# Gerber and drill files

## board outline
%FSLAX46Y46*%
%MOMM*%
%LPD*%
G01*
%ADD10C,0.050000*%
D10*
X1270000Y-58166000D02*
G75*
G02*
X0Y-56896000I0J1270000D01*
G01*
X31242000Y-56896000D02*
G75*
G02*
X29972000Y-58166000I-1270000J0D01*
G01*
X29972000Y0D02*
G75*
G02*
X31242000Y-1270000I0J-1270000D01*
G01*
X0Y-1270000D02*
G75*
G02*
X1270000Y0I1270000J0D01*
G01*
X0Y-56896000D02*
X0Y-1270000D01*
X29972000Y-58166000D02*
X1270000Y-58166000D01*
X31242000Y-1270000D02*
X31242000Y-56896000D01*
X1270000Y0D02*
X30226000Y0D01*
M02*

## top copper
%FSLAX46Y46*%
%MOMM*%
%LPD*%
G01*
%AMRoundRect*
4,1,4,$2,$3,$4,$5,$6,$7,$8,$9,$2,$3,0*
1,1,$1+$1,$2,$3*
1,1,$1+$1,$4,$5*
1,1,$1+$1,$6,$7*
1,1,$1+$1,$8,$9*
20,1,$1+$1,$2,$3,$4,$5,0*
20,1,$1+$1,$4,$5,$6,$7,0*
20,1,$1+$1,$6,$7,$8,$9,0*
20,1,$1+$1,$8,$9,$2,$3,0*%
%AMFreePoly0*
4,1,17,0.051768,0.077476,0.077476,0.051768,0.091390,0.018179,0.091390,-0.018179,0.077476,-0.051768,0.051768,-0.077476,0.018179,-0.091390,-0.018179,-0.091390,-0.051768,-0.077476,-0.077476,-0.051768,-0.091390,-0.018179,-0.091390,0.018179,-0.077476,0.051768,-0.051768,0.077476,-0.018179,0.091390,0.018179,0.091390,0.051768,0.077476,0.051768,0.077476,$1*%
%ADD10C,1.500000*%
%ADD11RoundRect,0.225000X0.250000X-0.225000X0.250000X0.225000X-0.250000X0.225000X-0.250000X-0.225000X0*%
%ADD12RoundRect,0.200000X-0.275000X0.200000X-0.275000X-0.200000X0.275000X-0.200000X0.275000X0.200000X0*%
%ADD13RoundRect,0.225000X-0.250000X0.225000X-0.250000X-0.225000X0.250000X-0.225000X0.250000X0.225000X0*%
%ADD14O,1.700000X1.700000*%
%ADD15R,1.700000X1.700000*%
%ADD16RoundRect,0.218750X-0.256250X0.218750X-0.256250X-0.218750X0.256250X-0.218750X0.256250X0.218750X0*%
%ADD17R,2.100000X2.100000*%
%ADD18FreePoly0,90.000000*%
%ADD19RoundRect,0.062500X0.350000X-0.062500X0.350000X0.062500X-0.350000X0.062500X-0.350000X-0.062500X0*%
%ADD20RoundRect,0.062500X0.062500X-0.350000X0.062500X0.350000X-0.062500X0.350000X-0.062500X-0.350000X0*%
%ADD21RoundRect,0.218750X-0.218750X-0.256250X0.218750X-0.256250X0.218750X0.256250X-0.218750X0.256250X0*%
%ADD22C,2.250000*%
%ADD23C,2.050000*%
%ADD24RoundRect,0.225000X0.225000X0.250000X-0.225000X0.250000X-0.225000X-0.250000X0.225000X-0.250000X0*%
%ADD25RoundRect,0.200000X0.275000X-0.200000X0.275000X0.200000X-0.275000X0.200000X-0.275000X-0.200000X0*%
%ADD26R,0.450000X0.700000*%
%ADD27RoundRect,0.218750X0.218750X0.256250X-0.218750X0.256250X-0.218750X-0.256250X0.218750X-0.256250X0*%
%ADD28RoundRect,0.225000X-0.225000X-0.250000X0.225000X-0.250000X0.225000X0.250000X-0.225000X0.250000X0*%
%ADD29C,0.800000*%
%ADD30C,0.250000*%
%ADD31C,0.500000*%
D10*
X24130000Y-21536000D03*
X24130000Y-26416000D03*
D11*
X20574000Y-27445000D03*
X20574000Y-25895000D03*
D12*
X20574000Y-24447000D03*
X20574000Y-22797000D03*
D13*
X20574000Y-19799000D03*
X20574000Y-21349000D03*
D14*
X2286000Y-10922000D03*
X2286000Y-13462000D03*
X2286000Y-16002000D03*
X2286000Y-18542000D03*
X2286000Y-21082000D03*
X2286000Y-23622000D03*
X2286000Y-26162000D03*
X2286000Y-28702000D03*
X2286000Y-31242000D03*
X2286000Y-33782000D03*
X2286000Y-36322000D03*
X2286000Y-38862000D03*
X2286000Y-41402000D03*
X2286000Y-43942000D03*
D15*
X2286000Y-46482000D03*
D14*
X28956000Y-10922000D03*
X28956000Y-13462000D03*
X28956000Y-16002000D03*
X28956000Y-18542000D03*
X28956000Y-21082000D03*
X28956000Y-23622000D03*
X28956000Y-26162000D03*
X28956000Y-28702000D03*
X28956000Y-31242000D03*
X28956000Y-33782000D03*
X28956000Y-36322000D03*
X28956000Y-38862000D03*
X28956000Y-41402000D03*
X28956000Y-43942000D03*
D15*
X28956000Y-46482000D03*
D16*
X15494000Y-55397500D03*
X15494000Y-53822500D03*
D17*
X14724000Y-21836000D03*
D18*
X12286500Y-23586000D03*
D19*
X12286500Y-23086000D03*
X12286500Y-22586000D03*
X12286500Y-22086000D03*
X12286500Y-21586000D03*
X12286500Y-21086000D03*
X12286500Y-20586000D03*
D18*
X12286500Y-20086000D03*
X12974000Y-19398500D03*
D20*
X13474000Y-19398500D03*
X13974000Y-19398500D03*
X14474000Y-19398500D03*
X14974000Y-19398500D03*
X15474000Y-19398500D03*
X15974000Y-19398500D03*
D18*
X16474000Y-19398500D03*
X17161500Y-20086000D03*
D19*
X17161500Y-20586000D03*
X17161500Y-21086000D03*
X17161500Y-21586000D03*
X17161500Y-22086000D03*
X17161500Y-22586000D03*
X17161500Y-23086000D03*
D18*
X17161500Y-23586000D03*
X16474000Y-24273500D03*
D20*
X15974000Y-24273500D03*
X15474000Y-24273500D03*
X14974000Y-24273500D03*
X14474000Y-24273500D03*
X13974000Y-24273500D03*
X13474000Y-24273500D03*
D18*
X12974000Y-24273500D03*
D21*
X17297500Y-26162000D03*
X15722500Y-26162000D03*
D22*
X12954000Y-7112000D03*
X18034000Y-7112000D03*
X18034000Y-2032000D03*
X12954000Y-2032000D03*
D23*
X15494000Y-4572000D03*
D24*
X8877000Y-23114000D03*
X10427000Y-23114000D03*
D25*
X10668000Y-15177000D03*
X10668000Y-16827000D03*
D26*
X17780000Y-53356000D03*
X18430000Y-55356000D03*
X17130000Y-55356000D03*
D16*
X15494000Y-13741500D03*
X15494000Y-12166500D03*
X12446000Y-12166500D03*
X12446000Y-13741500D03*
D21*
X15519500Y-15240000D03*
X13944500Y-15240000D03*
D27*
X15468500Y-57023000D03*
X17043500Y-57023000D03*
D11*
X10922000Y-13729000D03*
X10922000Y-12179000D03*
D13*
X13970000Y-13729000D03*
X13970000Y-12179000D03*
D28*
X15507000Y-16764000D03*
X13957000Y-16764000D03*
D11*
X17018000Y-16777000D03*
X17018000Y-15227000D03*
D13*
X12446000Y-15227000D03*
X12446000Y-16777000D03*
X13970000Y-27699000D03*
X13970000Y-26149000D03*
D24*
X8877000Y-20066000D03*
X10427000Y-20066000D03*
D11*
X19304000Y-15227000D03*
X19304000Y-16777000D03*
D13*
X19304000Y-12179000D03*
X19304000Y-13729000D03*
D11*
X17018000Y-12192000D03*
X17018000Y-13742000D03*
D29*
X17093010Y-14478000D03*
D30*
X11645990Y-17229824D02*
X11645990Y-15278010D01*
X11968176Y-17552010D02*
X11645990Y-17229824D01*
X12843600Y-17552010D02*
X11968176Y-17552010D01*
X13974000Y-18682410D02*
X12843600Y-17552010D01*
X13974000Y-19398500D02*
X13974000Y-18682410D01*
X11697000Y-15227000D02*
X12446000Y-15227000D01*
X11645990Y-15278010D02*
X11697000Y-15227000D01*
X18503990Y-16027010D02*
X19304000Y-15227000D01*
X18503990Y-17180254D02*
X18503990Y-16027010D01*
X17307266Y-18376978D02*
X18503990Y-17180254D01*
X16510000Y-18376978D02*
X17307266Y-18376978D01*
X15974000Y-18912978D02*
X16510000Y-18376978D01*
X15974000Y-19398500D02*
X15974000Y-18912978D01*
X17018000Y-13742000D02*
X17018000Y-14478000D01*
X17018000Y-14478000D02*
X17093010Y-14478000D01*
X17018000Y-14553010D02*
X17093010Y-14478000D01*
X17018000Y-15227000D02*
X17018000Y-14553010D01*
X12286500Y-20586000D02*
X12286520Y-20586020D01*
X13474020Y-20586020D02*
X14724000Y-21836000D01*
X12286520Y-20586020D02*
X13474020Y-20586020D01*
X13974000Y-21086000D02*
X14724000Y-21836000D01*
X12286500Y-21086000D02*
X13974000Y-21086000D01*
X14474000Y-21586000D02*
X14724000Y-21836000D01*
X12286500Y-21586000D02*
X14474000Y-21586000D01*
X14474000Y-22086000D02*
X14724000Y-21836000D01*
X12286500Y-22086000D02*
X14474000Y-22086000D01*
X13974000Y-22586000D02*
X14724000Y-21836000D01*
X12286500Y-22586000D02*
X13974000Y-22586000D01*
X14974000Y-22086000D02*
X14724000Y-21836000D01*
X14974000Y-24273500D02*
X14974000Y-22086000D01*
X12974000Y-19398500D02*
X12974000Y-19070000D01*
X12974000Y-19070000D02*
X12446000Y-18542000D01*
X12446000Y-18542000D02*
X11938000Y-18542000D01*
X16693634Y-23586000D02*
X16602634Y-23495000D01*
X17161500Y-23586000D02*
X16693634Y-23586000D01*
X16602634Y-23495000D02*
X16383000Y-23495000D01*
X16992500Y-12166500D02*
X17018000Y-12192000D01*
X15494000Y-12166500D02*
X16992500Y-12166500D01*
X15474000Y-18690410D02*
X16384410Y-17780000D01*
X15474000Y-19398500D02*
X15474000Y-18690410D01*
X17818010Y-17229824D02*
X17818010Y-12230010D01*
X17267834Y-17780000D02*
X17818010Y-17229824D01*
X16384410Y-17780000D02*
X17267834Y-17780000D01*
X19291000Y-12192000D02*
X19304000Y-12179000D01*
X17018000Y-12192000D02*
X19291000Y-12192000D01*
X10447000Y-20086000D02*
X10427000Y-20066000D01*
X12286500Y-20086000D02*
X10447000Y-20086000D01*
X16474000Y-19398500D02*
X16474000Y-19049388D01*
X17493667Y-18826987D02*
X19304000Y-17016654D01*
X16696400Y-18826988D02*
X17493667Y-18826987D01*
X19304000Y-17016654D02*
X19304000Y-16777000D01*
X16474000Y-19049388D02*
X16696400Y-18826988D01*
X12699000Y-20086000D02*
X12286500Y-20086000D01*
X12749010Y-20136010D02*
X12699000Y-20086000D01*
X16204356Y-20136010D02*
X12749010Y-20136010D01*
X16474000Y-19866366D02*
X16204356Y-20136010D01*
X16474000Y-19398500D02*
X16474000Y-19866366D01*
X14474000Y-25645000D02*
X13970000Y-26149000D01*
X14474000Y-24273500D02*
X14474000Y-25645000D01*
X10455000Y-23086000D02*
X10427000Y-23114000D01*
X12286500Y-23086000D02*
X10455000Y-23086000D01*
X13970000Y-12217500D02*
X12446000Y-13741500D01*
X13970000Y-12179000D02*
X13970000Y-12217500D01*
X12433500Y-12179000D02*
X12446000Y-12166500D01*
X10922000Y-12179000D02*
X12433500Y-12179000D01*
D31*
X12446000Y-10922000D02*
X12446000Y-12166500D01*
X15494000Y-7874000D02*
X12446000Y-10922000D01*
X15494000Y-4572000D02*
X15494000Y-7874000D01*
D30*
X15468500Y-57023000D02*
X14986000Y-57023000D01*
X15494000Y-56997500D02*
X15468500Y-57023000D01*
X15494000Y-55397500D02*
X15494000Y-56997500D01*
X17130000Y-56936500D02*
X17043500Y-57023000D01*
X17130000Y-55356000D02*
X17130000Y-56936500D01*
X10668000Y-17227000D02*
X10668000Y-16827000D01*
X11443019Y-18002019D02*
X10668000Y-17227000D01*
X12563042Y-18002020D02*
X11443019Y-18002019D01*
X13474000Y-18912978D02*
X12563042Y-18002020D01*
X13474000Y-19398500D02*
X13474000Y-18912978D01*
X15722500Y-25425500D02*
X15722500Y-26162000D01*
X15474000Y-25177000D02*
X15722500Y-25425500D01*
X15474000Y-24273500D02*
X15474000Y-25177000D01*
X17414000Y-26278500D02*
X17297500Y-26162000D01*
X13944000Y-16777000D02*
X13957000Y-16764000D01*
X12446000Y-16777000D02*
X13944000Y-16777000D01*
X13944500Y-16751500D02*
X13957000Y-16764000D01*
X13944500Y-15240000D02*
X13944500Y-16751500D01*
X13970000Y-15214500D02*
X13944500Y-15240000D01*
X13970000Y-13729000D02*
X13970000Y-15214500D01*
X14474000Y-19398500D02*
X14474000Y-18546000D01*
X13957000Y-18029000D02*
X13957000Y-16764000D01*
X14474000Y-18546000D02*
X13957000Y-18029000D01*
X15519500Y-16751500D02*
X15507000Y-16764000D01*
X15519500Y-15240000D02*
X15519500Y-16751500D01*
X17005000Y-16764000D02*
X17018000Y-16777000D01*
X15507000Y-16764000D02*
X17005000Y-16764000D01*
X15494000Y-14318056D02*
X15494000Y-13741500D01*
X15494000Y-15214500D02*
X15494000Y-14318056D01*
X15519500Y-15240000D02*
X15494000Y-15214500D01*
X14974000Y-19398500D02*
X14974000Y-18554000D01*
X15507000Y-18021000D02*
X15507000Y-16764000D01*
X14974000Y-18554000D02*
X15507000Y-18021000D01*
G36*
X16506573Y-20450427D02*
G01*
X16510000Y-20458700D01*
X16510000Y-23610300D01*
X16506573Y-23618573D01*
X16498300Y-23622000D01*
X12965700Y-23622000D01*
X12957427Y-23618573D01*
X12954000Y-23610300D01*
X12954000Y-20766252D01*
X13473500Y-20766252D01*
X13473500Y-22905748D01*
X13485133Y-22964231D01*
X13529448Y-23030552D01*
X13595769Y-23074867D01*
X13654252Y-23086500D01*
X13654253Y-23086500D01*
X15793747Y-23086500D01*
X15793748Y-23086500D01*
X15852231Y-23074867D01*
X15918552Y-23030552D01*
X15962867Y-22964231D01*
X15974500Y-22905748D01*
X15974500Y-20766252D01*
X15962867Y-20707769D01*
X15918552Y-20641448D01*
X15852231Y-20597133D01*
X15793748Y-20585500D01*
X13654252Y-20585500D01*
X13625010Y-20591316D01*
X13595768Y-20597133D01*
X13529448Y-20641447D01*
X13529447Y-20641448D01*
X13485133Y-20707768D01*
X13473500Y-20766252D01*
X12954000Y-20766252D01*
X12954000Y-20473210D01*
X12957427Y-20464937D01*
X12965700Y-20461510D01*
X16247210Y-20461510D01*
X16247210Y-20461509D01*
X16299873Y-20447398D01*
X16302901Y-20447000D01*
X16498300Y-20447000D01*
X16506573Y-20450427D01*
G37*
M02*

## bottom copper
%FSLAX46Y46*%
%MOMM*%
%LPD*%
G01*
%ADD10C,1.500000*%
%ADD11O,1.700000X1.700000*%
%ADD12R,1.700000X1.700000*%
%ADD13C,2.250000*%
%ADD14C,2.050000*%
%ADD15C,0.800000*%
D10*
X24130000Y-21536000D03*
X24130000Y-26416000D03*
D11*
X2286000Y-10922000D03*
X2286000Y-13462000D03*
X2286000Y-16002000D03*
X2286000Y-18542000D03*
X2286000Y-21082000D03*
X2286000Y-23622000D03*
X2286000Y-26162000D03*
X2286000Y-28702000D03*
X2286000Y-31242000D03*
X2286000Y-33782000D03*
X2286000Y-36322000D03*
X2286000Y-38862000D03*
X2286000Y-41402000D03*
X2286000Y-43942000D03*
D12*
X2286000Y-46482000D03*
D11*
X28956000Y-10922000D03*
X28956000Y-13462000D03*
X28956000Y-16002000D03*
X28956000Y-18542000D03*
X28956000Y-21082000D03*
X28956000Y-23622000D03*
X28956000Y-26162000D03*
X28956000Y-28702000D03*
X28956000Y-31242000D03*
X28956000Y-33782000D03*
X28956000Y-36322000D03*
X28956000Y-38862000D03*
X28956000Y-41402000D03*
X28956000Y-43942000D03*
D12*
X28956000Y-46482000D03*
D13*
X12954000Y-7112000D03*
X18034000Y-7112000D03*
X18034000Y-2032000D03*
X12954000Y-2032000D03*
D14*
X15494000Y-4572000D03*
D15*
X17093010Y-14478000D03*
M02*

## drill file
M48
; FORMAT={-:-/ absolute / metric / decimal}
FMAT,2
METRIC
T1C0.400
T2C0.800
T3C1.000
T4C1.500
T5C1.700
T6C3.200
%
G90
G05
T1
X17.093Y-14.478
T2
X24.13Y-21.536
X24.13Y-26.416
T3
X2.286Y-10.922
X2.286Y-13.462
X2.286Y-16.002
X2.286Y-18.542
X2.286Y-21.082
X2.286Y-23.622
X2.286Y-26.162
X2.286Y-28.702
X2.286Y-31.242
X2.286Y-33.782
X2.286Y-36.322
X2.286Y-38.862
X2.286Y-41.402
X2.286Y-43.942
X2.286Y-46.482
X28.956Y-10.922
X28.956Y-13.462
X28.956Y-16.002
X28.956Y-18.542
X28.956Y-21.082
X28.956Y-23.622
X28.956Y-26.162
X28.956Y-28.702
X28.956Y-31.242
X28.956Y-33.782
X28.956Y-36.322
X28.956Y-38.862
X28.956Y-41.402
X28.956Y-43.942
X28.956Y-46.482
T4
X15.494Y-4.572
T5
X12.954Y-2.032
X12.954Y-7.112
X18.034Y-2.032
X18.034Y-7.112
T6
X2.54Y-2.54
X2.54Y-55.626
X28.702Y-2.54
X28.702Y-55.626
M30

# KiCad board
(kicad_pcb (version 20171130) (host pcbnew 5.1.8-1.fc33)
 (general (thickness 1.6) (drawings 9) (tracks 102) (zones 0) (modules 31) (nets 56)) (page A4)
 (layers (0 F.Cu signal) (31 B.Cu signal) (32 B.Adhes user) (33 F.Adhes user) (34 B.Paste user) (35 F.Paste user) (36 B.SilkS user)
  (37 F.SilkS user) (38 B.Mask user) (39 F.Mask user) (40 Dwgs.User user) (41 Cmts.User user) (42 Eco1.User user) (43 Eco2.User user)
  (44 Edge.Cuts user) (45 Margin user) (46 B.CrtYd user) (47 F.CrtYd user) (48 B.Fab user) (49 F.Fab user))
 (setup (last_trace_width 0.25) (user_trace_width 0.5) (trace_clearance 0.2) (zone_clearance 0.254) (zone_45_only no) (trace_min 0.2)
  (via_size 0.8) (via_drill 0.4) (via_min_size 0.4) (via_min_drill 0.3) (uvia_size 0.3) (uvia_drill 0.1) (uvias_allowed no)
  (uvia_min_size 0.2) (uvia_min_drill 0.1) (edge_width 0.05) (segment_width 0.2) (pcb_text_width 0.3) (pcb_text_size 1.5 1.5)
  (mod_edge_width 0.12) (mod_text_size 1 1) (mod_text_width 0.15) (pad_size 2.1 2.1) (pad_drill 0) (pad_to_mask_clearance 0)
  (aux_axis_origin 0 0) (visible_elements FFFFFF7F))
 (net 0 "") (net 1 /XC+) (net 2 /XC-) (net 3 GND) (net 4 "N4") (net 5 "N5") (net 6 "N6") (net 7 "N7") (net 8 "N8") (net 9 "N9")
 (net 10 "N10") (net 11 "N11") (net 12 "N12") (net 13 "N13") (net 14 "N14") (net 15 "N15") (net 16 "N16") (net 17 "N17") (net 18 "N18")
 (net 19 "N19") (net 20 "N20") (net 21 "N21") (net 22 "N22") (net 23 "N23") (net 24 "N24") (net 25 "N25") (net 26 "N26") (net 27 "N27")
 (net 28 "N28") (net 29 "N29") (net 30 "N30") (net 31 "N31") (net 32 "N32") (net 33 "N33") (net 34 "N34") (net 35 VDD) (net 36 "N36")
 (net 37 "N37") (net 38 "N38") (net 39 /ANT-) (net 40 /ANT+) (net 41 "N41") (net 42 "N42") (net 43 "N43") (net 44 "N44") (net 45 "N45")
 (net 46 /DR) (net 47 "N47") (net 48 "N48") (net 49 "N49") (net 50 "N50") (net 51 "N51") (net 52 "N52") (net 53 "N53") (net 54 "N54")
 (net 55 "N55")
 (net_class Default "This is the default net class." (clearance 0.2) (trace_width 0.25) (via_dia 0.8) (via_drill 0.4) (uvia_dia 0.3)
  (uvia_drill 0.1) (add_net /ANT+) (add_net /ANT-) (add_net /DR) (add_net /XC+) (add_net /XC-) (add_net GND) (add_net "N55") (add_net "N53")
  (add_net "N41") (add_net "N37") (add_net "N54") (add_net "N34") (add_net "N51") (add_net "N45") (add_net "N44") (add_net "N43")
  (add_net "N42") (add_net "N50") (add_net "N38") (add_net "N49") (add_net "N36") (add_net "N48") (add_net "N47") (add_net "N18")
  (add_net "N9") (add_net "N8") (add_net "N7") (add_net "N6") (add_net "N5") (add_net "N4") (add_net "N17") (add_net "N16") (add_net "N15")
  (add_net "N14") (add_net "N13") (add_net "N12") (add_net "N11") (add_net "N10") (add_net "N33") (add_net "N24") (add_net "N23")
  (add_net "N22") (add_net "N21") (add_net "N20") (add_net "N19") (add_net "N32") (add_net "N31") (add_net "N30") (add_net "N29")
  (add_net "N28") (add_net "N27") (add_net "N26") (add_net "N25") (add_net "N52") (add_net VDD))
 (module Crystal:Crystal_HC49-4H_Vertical (layer F.Cu) (at 24.13 26.416 90)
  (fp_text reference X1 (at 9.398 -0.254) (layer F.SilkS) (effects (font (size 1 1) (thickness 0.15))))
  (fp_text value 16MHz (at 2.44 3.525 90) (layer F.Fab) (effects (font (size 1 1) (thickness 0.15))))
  (pad 2 thru_hole circle (at 4.88 0 90) (size 1.5 1.5) (drill 0.8) (layers *.Cu *.Mask) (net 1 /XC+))
  (pad 1 thru_hole circle (at 0 0 90) (size 1.5 1.5) (drill 0.8) (layers *.Cu *.Mask) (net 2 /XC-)))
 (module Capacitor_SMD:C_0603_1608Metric (layer F.Cu) (at 20.574 26.67 90)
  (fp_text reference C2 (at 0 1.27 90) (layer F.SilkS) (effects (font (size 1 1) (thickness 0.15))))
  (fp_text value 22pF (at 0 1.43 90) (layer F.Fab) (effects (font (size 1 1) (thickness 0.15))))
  (pad 1 smd roundrect (at -0.775 0 90) (size 0.9 0.95) (layers F.Cu F.Paste F.Mask) (roundrect_rratio 0.25) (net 1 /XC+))
  (pad 2 smd roundrect (at 0.775 0 90) (size 0.9 0.95) (layers F.Cu F.Paste F.Mask) (roundrect_rratio 0.25) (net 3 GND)))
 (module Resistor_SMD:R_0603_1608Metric (layer F.Cu) (at 20.574 23.622 270)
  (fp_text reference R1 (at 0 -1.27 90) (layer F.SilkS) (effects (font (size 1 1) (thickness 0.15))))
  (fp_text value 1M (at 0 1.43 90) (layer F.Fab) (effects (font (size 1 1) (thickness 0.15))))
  (pad 2 smd roundrect (at 0.825 0 270) (size 0.8 0.95) (layers F.Cu F.Paste F.Mask) (roundrect_rratio 0.25) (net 2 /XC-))
  (pad 1 smd roundrect (at -0.825 0 270) (size 0.8 0.95) (layers F.Cu F.Paste F.Mask) (roundrect_rratio 0.25) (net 1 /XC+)))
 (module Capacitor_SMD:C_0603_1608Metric (layer F.Cu) (at 20.574 20.574 270)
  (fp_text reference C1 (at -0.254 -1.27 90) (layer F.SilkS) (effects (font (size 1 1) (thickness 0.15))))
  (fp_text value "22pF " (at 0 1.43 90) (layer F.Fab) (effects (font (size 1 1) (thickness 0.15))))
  (pad 1 smd roundrect (at -0.775 0 270) (size 0.9 0.95) (layers F.Cu F.Paste F.Mask) (roundrect_rratio 0.25) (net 2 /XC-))
  (pad 2 smd roundrect (at 0.775 0 270) (size 0.9 0.95) (layers F.Cu F.Paste F.Mask) (roundrect_rratio 0.25) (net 3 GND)))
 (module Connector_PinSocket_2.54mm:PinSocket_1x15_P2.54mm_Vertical (layer F.Cu) (at 2.286 46.482 180)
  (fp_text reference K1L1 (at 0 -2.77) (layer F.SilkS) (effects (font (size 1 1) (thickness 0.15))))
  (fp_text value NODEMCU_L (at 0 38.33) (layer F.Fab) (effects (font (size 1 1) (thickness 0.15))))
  (pad 15 thru_hole oval (at 0 35.56 180) (size 1.7 1.7) (drill 1) (layers *.Cu *.Mask) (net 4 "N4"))
  (pad 14 thru_hole oval (at 0 33.02 180) (size 1.7 1.7) (drill 1) (layers *.Cu *.Mask) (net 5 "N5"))
  (pad 13 thru_hole oval (at 0 30.48 180) (size 1.7 1.7) (drill 1) (layers *.Cu *.Mask) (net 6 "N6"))
  (pad 12 thru_hole oval (at 0 27.94 180) (size 1.7 1.7) (drill 1) (layers *.Cu *.Mask) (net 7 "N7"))
  (pad 11 thru_hole oval (at 0 25.4 180) (size 1.7 1.7) (drill 1) (layers *.Cu *.Mask) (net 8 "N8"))
  (pad 10 thru_hole oval (at 0 22.86 180) (size 1.7 1.7) (drill 1) (layers *.Cu *.Mask) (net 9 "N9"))
  (pad 9 thru_hole oval (at 0 20.32 180) (size 1.7 1.7) (drill 1) (layers *.Cu *.Mask) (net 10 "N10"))
  (pad 8 thru_hole oval (at 0 17.78 180) (size 1.7 1.7) (drill 1) (layers *.Cu *.Mask) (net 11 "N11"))
  (pad 7 thru_hole oval (at 0 15.24 180) (size 1.7 1.7) (drill 1) (layers *.Cu *.Mask) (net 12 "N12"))
  (pad 6 thru_hole oval (at 0 12.7 180) (size 1.7 1.7) (drill 1) (layers *.Cu *.Mask) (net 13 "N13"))
  (pad 5 thru_hole oval (at 0 10.16 180) (size 1.7 1.7) (drill 1) (layers *.Cu *.Mask) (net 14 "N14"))
  (pad 4 thru_hole oval (at 0 7.62 180) (size 1.7 1.7) (drill 1) (layers *.Cu *.Mask) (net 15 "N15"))
  (pad 3 thru_hole oval (at 0 5.08 180) (size 1.7 1.7) (drill 1) (layers *.Cu *.Mask) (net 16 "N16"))
  (pad 2 thru_hole oval (at 0 2.54 180) (size 1.7 1.7) (drill 1) (layers *.Cu *.Mask) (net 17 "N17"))
  (pad 1 thru_hole rect (at 0 0 180) (size 1.7 1.7) (drill 1) (layers *.Cu *.Mask) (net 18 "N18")))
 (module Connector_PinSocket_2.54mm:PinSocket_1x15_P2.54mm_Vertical (layer F.Cu) (at 28.956 46.482 180)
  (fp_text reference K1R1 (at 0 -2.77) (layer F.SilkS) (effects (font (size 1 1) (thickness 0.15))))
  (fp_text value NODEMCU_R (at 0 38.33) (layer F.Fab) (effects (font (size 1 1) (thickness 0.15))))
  (pad 15 thru_hole oval (at 0 35.56 180) (size 1.7 1.7) (drill 1) (layers *.Cu *.Mask) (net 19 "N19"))
  (pad 14 thru_hole oval (at 0 33.02 180) (size 1.7 1.7) (drill 1) (layers *.Cu *.Mask) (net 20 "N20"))
  (pad 13 thru_hole oval (at 0 30.48 180) (size 1.7 1.7) (drill 1) (layers *.Cu *.Mask) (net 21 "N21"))
  (pad 12 thru_hole oval (at 0 27.94 180) (size 1.7 1.7) (drill 1) (layers *.Cu *.Mask) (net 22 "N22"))
  (pad 11 thru_hole oval (at 0 25.4 180) (size 1.7 1.7) (drill 1) (layers *.Cu *.Mask) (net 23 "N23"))
  (pad 10 thru_hole oval (at 0 22.86 180) (size 1.7 1.7) (drill 1) (layers *.Cu *.Mask) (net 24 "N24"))
  (pad 9 thru_hole oval (at 0 20.32 180) (size 1.7 1.7) (drill 1) (layers *.Cu *.Mask) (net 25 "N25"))
  (pad 8 thru_hole oval (at 0 17.78 180) (size 1.7 1.7) (drill 1) (layers *.Cu *.Mask) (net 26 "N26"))
  (pad 7 thru_hole oval (at 0 15.24 180) (size 1.7 1.7) (drill 1) (layers *.Cu *.Mask) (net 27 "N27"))
  (pad 6 thru_hole oval (at 0 12.7 180) (size 1.7 1.7) (drill 1) (layers *.Cu *.Mask) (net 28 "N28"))
  (pad 5 thru_hole oval (at 0 10.16 180) (size 1.7 1.7) (drill 1) (layers *.Cu *.Mask) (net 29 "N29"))
  (pad 4 thru_hole oval (at 0 7.62 180) (size 1.7 1.7) (drill 1) (layers *.Cu *.Mask) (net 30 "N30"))
  (pad 3 thru_hole oval (at 0 5.08 180) (size 1.7 1.7) (drill 1) (layers *.Cu *.Mask) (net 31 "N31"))
  (pad 2 thru_hole oval (at 0 2.54 180) (size 1.7 1.7) (drill 1) (layers *.Cu *.Mask) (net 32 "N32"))
  (pad 1 thru_hole rect (at 0 0 180) (size 1.7 1.7) (drill 1) (layers *.Cu *.Mask) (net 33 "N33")))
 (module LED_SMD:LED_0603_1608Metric (layer F.Cu) (at 15.494 54.61 270)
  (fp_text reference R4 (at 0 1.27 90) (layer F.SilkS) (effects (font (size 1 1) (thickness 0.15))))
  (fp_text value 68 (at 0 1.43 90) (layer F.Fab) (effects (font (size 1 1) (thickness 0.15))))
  (pad 2 smd roundrect (at 0.7875 0 270) (size 0.875 0.95) (layers F.Cu F.Paste F.Mask) (roundrect_rratio 0.25) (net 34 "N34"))
  (pad 1 smd roundrect (at -0.7875 0 270) (size 0.875 0.95) (layers F.Cu F.Paste F.Mask) (roundrect_rratio 0.25) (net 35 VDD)))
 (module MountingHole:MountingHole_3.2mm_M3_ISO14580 (layer F.Cu) (at 2.54 55.626)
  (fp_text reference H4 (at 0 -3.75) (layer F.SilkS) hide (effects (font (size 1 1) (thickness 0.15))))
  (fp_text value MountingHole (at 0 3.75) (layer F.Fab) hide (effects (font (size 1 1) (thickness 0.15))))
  (pad 1 np_thru_hole circle (at 0 0) (size 3.2 3.2) (drill 3.2) (layers *.Cu *.Mask)))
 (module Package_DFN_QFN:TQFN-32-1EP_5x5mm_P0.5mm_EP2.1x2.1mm (layer F.Cu) (at 14.724 21.836 90)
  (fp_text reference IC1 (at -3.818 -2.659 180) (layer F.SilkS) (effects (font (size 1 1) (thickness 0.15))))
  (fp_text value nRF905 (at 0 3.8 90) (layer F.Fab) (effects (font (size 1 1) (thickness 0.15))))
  (pad "" smd roundrect (at 0.525 0.525 90) (size 0.85 0.85) (layers F.Paste) (roundrect_rratio 0.25))
  (pad "" smd roundrect (at 0.525 -0.525 90) (size 0.85 0.85) (layers F.Paste) (roundrect_rratio 0.25))
  (pad "" smd roundrect (at -0.525 0.525 90) (size 0.85 0.85) (layers F.Paste) (roundrect_rratio 0.25))
  (pad "" smd roundrect (at -0.525 -0.525 90) (size 0.85 0.85) (layers F.Paste) (roundrect_rratio 0.25))
  (pad 33 smd rect (at 0 0 90) (size 2.1 2.1) (layers F.Cu F.Mask))
  (pad 32 smd custom (at -1.75 -2.4375 90) (size 0.18636 0.18636) (layers F.Cu F.Paste F.Mask) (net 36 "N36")
   (options (clearance outline) (anchor circle)) (primitives))
  (pad 31 smd roundrect (at -1.25 -2.4375 90) (size 0.25 0.825) (layers F.Cu F.Paste F.Mask) (roundrect_rratio 0.25) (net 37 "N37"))
  (pad 30 smd roundrect (at -0.75 -2.4375 90) (size 0.25 0.825) (layers F.Cu F.Paste F.Mask) (roundrect_rratio 0.25) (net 3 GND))
  (pad 29 smd roundrect (at -0.25 -2.4375 90) (size 0.25 0.825) (layers F.Cu F.Paste F.Mask) (roundrect_rratio 0.25) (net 3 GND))
  (pad 28 smd roundrect (at 0.25 -2.4375 90) (size 0.25 0.825) (layers F.Cu F.Paste F.Mask) (roundrect_rratio 0.25) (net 3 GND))
  (pad 27 smd roundrect (at 0.75 -2.4375 90) (size 0.25 0.825) (layers F.Cu F.Paste F.Mask) (roundrect_rratio 0.25) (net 3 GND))
  (pad 26 smd roundrect (at 1.25 -2.4375 90) (size 0.25 0.825) (layers F.Cu F.Paste F.Mask) (roundrect_rratio 0.25) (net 3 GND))
  (pad 25 smd custom (at 1.75 -2.4375 90) (size 0.18636 0.18636) (layers F.Cu F.Paste F.Mask) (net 35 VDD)
   (options (clearance outline) (anchor circle)) (primitives))
  (pad 24 smd custom (at 2.4375 -1.75 90) (size 0.18636 0.18636) (layers F.Cu F.Paste F.Mask) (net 3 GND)
   (options (clearance outline) (anchor circle)) (primitives))
  (pad 23 smd roundrect (at 2.4375 -1.25 90) (size 0.825 0.25) (layers F.Cu F.Paste F.Mask) (roundrect_rratio 0.25) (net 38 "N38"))
  (pad 22 smd roundrect (at 2.4375 -0.75 90) (size 0.825 0.25) (layers F.Cu F.Paste F.Mask) (roundrect_rratio 0.25) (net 3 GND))
  (pad 21 smd roundrect (at 2.4375 -0.25 90) (size 0.825 0.25) (layers F.Cu F.Paste F.Mask) (roundrect_rratio 0.25) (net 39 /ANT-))
  (pad 20 smd roundrect (at 2.4375 0.25 90) (size 0.825 0.25) (layers F.Cu F.Paste F.Mask) (roundrect_rratio 0.25) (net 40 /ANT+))
  (pad 19 smd roundrect (at 2.4375 0.75 90) (size 0.825 0.25) (layers F.Cu F.Paste F.Mask) (roundrect_rratio 0.25) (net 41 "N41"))
  (pad 18 smd roundrect (at 2.4375 1.25 90) (size 0.825 0.25) (layers F.Cu F.Paste F.Mask) (roundrect_rratio 0.25) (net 3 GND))
  (pad 17 smd custom (at 2.4375 1.75 90) (size 0.18636 0.18636) (layers F.Cu F.Paste F.Mask) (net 35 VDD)
   (options (clearance outline) (anchor circle)) (primitives))
  (pad 16 smd custom (at 1.75 2.4375 90) (size 0.18636 0.18636) (layers F.Cu F.Paste F.Mask) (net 3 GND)
   (options (clearance outline) (anchor circle)) (primitives))
  (pad 15 smd roundrect (at 1.25 2.4375 90) (size 0.25 0.825) (layers F.Cu F.Paste F.Mask) (roundrect_rratio 0.25) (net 2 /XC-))
  (pad 14 smd roundrect (at 0.75 2.4375 90) (size 0.25 0.825) (layers F.Cu F.Paste F.Mask) (roundrect_rratio 0.25) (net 1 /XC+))
  (pad 13 smd roundrect (at 0.25 2.4375 90) (size 0.25 0.825) (layers F.Cu F.Paste F.Mask) (roundrect_rratio 0.25) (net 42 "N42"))
  (pad 12 smd roundrect (at -0.25 2.4375 90) (size 0.25 0.825) (layers F.Cu F.Paste F.Mask) (roundrect_rratio 0.25) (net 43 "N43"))
  (pad 11 smd roundrect (at -0.75 2.4375 90) (size 0.25 0.825) (layers F.Cu F.Paste F.Mask) (roundrect_rratio 0.25) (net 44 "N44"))
  (pad 10 smd roundrect (at -1.25 2.4375 90) (size 0.25 0.825) (layers F.Cu F.Paste F.Mask) (roundrect_rratio 0.25) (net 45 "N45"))
  (pad 9 smd custom (at -1.75 2.4375 90) (size 0.18636 0.18636) (layers F.Cu F.Paste F.Mask) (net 3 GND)
   (options (clearance outline) (anchor circle)) (primitives))
  (pad 8 smd custom (at -2.4375 1.75 90) (size 0.18636 0.18636) (layers F.Cu F.Paste F.Mask) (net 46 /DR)
   (options (clearance outline) (anchor circle)) (primitives))
  (pad 7 smd roundrect (at -2.4375 1.25 90) (size 0.825 0.25) (layers F.Cu F.Paste F.Mask) (roundrect_rratio 0.25) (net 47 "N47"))
  (pad 6 smd roundrect (at -2.4375 0.75 90) (size 0.825 0.25) (layers F.Cu F.Paste F.Mask) (roundrect_rratio 0.25) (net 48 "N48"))
  (pad 5 smd roundrect (at -2.4375 0.25 90) (size 0.825 0.25) (layers F.Cu F.Paste F.Mask) (roundrect_rratio 0.25) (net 3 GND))
  (pad 4 smd roundrect (at -2.4375 -0.25 90) (size 0.825 0.25) (layers F.Cu F.Paste F.Mask) (roundrect_rratio 0.25) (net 35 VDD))
  (pad 3 smd roundrect (at -2.4375 -0.75 90) (size 0.825 0.25) (layers F.Cu F.Paste F.Mask) (roundrect_rratio 0.25) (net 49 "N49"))
  (pad 2 smd roundrect (at -2.4375 -1.25 90) (size 0.825 0.25) (layers F.Cu F.Paste F.Mask) (roundrect_rratio 0.25) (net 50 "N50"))
  (pad 1 smd custom (at -2.4375 -1.75 90) (size 0.18636 0.18636) (layers F.Cu F.Paste F.Mask) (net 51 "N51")
   (options (clearance outline) (anchor circle)) (primitives)))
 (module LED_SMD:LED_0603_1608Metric (layer F.Cu) (at 16.51 26.162)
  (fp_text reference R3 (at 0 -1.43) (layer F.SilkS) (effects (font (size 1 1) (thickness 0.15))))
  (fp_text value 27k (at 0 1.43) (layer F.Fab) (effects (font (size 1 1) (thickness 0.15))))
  (pad 2 smd roundrect (at 0.7875 0) (size 0.875 0.95) (layers F.Cu F.Paste F.Mask) (roundrect_rratio 0.25) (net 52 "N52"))
  (pad 1 smd roundrect (at -0.7875 0) (size 0.875 0.95) (layers F.Cu F.Paste F.Mask) (roundrect_rratio 0.25) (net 48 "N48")))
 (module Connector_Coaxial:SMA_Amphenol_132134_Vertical (layer B.Cu) (at 15.494 4.572 90)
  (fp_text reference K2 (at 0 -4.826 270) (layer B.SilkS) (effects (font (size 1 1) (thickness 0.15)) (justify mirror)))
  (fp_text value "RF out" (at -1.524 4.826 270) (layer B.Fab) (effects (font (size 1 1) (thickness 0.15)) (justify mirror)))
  (pad 2 thru_hole circle (at -2.54 -2.54 90) (size 2.25 2.25) (drill 1.7) (layers *.Cu *.Mask) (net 3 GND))
  (pad 2 thru_hole circle (at -2.54 2.54 90) (size 2.25 2.25) (drill 1.7) (layers *.Cu *.Mask) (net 3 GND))
  (pad 2 thru_hole circle (at 2.54 2.54 90) (size 2.25 2.25) (drill 1.7) (layers *.Cu *.Mask) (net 3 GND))
  (pad 2 thru_hole circle (at 2.54 -2.54 90) (size 2.25 2.25) (drill 1.7) (layers *.Cu *.Mask) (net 3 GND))
  (pad 1 thru_hole circle (at 0 0 90) (size 2.05 2.05) (drill 1.5) (layers *.Cu *.Mask) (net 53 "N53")))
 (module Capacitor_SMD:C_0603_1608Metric (layer F.Cu) (at 9.652 23.114 180)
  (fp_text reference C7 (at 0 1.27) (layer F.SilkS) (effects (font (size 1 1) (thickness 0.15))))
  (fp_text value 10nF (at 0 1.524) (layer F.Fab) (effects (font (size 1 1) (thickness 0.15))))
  (pad 2 smd roundrect (at 0.775 0 180) (size 0.9 0.95) (layers F.Cu F.Paste F.Mask) (roundrect_rratio 0.25) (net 3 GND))
  (pad 1 smd roundrect (at -0.775 0 180) (size 0.9 0.95) (layers F.Cu F.Paste F.Mask) (roundrect_rratio 0.25) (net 37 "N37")))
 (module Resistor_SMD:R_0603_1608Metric (layer F.Cu) (at 10.668 16.002 90)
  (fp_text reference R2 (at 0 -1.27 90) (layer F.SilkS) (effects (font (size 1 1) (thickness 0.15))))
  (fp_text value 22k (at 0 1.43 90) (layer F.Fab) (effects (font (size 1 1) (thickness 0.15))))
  (pad 2 smd roundrect (at 0.825 0 90) (size 0.8 0.95) (layers F.Cu F.Paste F.Mask) (roundrect_rratio 0.25) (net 3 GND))
  (pad 1 smd roundrect (at -0.825 0 90) (size 0.8 0.95) (layers F.Cu F.Paste F.Mask) (roundrect_rratio 0.25) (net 38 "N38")))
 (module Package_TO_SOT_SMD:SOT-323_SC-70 (layer F.Cu) (at 17.78 54.356 90)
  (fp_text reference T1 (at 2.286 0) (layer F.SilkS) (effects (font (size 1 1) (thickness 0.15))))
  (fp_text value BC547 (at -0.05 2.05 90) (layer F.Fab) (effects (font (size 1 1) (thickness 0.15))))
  (pad 3 smd rect (at 1 0) (size 0.45 0.7) (layers F.Cu F.Paste F.Mask) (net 3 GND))
  (pad 2 smd rect (at -1 0.65) (size 0.45 0.7) (layers F.Cu F.Paste F.Mask) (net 52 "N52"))
  (pad 1 smd rect (at -1 -0.65) (size 0.45 0.7) (layers F.Cu F.Paste F.Mask) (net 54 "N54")))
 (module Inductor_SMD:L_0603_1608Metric (layer F.Cu) (at 15.494 12.954 270)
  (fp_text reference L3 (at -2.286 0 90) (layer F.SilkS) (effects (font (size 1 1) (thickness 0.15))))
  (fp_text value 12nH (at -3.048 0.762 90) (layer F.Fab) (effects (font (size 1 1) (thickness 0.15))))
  (pad 2 smd roundrect (at 0.7875 0 270) (size 0.875 0.95) (layers F.Cu F.Paste F.Mask) (roundrect_rratio 0.25) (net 40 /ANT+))
  (pad 1 smd roundrect (at -0.7875 0 270) (size 0.875 0.95) (layers F.Cu F.Paste F.Mask) (roundrect_rratio 0.25) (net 41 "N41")))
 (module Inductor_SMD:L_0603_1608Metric (layer F.Cu) (at 12.446 12.954 270)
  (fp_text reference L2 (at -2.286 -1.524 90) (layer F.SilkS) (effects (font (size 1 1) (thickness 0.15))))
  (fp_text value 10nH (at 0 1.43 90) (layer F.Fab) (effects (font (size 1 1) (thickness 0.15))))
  (pad 1 smd roundrect (at -0.7875 0 270) (size 0.875 0.95) (layers F.Cu F.Paste F.Mask) (roundrect_rratio 0.25) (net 53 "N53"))
  (pad 2 smd roundrect (at 0.7875 0 270) (size 0.875 0.95) (layers F.Cu F.Paste F.Mask) (roundrect_rratio 0.25) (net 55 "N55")))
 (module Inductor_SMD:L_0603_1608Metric (layer F.Cu) (at 14.732 15.24)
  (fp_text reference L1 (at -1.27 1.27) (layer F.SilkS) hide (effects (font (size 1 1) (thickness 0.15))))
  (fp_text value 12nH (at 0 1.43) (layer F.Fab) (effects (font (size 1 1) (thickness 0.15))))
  (pad 2 smd roundrect (at 0.7875 0) (size 0.875 0.95) (layers F.Cu F.Paste F.Mask) (roundrect_rratio 0.25) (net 40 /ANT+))
  (pad 1 smd roundrect (at -0.7875 0) (size 0.875 0.95) (layers F.Cu F.Paste F.Mask) (roundrect_rratio 0.25) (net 39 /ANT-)))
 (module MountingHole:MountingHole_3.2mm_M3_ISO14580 (layer F.Cu) (at 28.702 55.626)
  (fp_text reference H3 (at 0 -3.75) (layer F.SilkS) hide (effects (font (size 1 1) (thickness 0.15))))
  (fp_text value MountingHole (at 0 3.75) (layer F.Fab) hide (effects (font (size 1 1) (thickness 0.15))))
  (pad 1 np_thru_hole circle (at 0 0) (size 3.2 3.2) (drill 3.2) (layers *.Cu *.Mask)))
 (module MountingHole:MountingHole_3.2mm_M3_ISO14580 (layer F.Cu) (at 28.702 2.54)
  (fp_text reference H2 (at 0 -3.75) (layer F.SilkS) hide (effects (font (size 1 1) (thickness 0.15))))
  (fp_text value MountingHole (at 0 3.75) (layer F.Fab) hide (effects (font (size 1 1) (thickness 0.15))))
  (pad 1 np_thru_hole circle (at 0 0) (size 3.2 3.2) (drill 3.2) (layers *.Cu *.Mask)))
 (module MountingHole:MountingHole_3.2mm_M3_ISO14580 (layer F.Cu) (at 2.54 2.54)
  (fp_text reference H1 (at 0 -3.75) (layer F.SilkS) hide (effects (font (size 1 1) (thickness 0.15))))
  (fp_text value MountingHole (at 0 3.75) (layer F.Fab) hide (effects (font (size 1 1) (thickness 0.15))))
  (pad 1 np_thru_hole circle (at 0 0) (size 3.2 3.2) (drill 3.2) (layers *.Cu *.Mask)))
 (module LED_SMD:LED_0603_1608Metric (layer F.Cu) (at 16.256 57.023 180)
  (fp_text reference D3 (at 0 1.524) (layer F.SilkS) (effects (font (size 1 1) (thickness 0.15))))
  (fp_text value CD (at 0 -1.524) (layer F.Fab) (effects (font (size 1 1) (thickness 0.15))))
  (pad 2 smd roundrect (at 0.7875 0 180) (size 0.875 0.95) (layers F.Cu F.Paste F.Mask) (roundrect_rratio 0.25) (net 34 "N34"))
  (pad 1 smd roundrect (at -0.7875 0 180) (size 0.875 0.95) (layers F.Cu F.Paste F.Mask) (roundrect_rratio 0.25) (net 54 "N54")))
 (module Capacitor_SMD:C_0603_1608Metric (layer F.Cu) (at 10.922 12.954 90)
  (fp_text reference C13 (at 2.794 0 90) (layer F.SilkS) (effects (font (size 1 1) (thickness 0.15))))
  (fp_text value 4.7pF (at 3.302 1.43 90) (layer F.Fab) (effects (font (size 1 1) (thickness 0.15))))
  (pad 1 smd roundrect (at -0.775 0 90) (size 0.9 0.95) (layers F.Cu F.Paste F.Mask) (roundrect_rratio 0.25) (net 3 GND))
  (pad 2 smd roundrect (at 0.775 0 90) (size 0.9 0.95) (layers F.Cu F.Paste F.Mask) (roundrect_rratio 0.25) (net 53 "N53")))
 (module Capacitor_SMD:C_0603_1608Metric (layer F.Cu) (at 13.97 12.954 270)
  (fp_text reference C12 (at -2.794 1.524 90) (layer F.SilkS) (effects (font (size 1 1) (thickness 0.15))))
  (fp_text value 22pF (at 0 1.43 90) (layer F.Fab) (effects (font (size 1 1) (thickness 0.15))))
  (pad 2 smd roundrect (at 0.775 0 270) (size 0.9 0.95) (layers F.Cu F.Paste F.Mask) (roundrect_rratio 0.25) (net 39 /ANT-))
  (pad 1 smd roundrect (at -0.775 0 270) (size 0.9 0.95) (layers F.Cu F.Paste F.Mask) (roundrect_rratio 0.25) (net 55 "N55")))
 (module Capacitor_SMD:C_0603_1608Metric (layer F.Cu) (at 14.732 16.764)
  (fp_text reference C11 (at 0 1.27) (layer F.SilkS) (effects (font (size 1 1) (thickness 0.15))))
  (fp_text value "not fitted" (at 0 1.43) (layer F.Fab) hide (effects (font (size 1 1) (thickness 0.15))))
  (pad 2 smd roundrect (at 0.775 0) (size 0.9 0.95) (layers F.Cu F.Paste F.Mask) (roundrect_rratio 0.25) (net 40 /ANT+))
  (pad 1 smd roundrect (at -0.775 0) (size 0.9 0.95) (layers F.Cu F.Paste F.Mask) (roundrect_rratio 0.25) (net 39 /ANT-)))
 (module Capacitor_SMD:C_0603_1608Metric (layer F.Cu) (at 17.018 16.002 90)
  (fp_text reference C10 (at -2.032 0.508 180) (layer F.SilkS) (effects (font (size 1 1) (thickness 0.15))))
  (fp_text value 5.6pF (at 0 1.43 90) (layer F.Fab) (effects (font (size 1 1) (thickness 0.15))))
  (pad 1 smd roundrect (at -0.775 0 90) (size 0.9 0.95) (layers F.Cu F.Paste F.Mask) (roundrect_rratio 0.25) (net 40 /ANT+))
  (pad 2 smd roundrect (at 0.775 0 90) (size 0.9 0.95) (layers F.Cu F.Paste F.Mask) (roundrect_rratio 0.25) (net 3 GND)))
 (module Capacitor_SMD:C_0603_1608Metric (layer F.Cu) (at 12.446 16.002 270)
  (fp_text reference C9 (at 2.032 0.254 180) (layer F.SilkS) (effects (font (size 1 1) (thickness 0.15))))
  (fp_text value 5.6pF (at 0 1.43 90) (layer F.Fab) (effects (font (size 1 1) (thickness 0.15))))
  (pad 1 smd roundrect (at -0.775 0 270) (size 0.9 0.95) (layers F.Cu F.Paste F.Mask) (roundrect_rratio 0.25) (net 3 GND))
  (pad 2 smd roundrect (at 0.775 0 270) (size 0.9 0.95) (layers F.Cu F.Paste F.Mask) (roundrect_rratio 0.25) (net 39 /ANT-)))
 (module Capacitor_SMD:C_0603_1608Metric (layer F.Cu) (at 13.97 26.924 270)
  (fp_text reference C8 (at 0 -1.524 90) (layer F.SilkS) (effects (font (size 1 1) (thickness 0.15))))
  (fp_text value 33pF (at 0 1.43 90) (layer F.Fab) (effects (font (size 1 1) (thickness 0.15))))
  (pad 2 smd roundrect (at 0.775 0 270) (size 0.9 0.95) (layers F.Cu F.Paste F.Mask) (roundrect_rratio 0.25) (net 3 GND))
  (pad 1 smd roundrect (at -0.775 0 270) (size 0.9 0.95) (layers F.Cu F.Paste F.Mask) (roundrect_rratio 0.25) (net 35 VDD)))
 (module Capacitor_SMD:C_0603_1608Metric (layer F.Cu) (at 9.652 20.066 180)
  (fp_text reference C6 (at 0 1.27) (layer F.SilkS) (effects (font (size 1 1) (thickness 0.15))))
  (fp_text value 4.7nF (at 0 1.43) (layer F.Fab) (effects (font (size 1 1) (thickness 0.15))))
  (pad 2 smd roundrect (at 0.775 0 180) (size 0.9 0.95) (layers F.Cu F.Paste F.Mask) (roundrect_rratio 0.25) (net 3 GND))
  (pad 1 smd roundrect (at -0.775 0 180) (size 0.9 0.95) (layers F.Cu F.Paste F.Mask) (roundrect_rratio 0.25) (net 35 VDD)))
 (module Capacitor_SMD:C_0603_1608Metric (layer F.Cu) (at 19.304 16.002 90)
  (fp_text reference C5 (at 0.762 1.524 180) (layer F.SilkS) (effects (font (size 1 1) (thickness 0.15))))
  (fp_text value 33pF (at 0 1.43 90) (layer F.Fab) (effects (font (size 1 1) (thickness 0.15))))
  (pad 2 smd roundrect (at 0.775 0 90) (size 0.9 0.95) (layers F.Cu F.Paste F.Mask) (roundrect_rratio 0.25) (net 3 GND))
  (pad 1 smd roundrect (at -0.775 0 90) (size 0.9 0.95) (layers F.Cu F.Paste F.Mask) (roundrect_rratio 0.25) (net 35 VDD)))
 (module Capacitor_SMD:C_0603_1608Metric (layer F.Cu) (at 19.304 12.954 270)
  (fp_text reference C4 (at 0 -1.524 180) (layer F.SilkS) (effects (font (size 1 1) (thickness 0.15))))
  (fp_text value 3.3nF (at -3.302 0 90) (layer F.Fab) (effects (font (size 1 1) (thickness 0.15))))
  (pad 1 smd roundrect (at -0.775 0 270) (size 0.9 0.95) (layers F.Cu F.Paste F.Mask) (roundrect_rratio 0.25) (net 41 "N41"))
  (pad 2 smd roundrect (at 0.775 0 270) (size 0.9 0.95) (layers F.Cu F.Paste F.Mask) (roundrect_rratio 0.25) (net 3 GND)))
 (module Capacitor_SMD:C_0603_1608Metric (layer F.Cu) (at 17.018 12.967 90)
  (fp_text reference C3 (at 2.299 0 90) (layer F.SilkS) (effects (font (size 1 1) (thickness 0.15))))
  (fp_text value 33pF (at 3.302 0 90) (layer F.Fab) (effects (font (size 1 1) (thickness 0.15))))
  (pad 2 smd roundrect (at 0.775 0 90) (size 0.9 0.95) (layers F.Cu F.Paste F.Mask) (roundrect_rratio 0.25) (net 41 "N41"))
  (pad 1 smd roundrect (at -0.775 0 90) (size 0.9 0.95) (layers F.Cu F.Paste F.Mask) (roundrect_rratio 0.25) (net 3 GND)))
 (gr_arc (start 1.27 56.896) (end 0 56.896) (angle -90) (layer Edge.Cuts) (width 0.05))
 (gr_arc (start 29.972 56.896) (end 29.972 58.166) (angle -90) (layer Edge.Cuts) (width 0.05))
 (gr_arc (start 29.972 1.27) (end 31.242 1.27) (angle -90) (layer Edge.Cuts) (width 0.05))
 (gr_arc (start 1.27 1.27) (end 1.27 0) (angle -90) (layer Edge.Cuts) (width 0.05))
 (gr_line (start 0 56.896) (end 0 1.27) (layer Edge.Cuts) (width 0.05))
 (gr_line (start 29.972 58.166) (end 1.27 58.166) (layer Edge.Cuts) (width 0.05))
 (gr_line (start 31.242 1.27) (end 31.242 56.896) (layer Edge.Cuts) (width 0.05))
 (gr_line (start 1.27 0) (end 30.226 0) (layer Edge.Cuts) (width 0.05))
 (segment (start 11.64599 17.229824) (end 11.64599 15.27801) (width 0.25) (layer F.Cu) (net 3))
 (segment (start 11.968176 17.55201) (end 11.64599 17.229824) (width 0.25) (layer F.Cu) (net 3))
 (segment (start 12.8436 17.55201) (end 11.968176 17.55201) (width 0.25) (layer F.Cu) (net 3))
 (segment (start 13.974 18.68241) (end 12.8436 17.55201) (width 0.25) (layer F.Cu) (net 3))
 (segment (start 13.974 19.3985) (end 13.974 18.68241) (width 0.25) (layer F.Cu) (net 3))
 (segment (start 11.697 15.227) (end 12.446 15.227) (width 0.25) (layer F.Cu) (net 3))
 (segment (start 11.64599 15.27801) (end 11.697 15.227) (width 0.25) (layer F.Cu) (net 3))
 (segment (start 18.50399 16.02701) (end 19.304 15.227) (width 0.25) (layer F.Cu) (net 3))
 (segment (start 18.50399 17.180254) (end 18.50399 16.02701) (width 0.25) (layer F.Cu) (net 3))
 (segment (start 17.307266 18.376978) (end 18.50399 17.180254) (width 0.25) (layer F.Cu) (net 3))
 (segment (start 16.51 18.376978) (end 17.307266 18.376978) (width 0.25) (layer F.Cu) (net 3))
 (segment (start 15.974 18.912978) (end 16.51 18.376978) (width 0.25) (layer F.Cu) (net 3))
 (segment (start 15.974 19.3985) (end 15.974 18.912978) (width 0.25) (layer F.Cu) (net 3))
 (segment (start 17.018 13.742) (end 17.018 14.478) (width 0.25) (layer F.Cu) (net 3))
 (via (at 17.09301 14.478) (size 0.8) (drill 0.4) (layers F.Cu B.Cu) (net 3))
 (segment (start 17.018 14.478) (end 17.09301 14.478) (width 0.25) (layer F.Cu) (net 3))
 (segment (start 17.018 14.55301) (end 17.09301 14.478) (width 0.25) (layer F.Cu) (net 3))
 (segment (start 17.018 15.227) (end 17.018 14.55301) (width 0.25) (layer F.Cu) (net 3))
 (segment (start 12.2865 20.586) (end 12.28652 20.58602) (width 0.25) (layer F.Cu) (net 3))
 (segment (start 13.47402 20.58602) (end 14.724 21.836) (width 0.25) (layer F.Cu) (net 3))
 (segment (start 12.28652 20.58602) (end 13.47402 20.58602) (width 0.25) (layer F.Cu) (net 3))
 (segment (start 13.974 21.086) (end 14.724 21.836) (width 0.25) (layer F.Cu) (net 3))
 (segment (start 12.2865 21.086) (end 13.974 21.086) (width 0.25) (layer F.Cu) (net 3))
 (segment (start 14.474 21.586) (end 14.724 21.836) (width 0.25) (layer F.Cu) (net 3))
 (segment (start 12.2865 21.586) (end 14.474 21.586) (width 0.25) (layer F.Cu) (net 3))
 (segment (start 14.474 22.086) (end 14.724 21.836) (width 0.25) (layer F.Cu) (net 3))
 (segment (start 12.2865 22.086) (end 14.474 22.086) (width 0.25) (layer F.Cu) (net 3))
 (segment (start 13.974 22.586) (end 14.724 21.836) (width 0.25) (layer F.Cu) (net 3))
 (segment (start 12.2865 22.586) (end 13.974 22.586) (width 0.25) (layer F.Cu) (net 3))
 (segment (start 14.974 22.086) (end 14.724 21.836) (width 0.25) (layer F.Cu) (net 3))
 (segment (start 14.974 24.2735) (end 14.974 22.086) (width 0.25) (layer F.Cu) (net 3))
 (segment (start 12.974 19.3985) (end 12.974 19.07) (width 0.25) (layer F.Cu) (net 3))
 (segment (start 12.974 19.07) (end 12.446 18.542) (width 0.25) (layer F.Cu) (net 3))
 (segment (start 12.446 18.542) (end 11.938 18.542) (width 0.25) (layer F.Cu) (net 3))
 (segment (start 16.693634 23.586) (end 16.602634 23.495) (width 0.25) (layer F.Cu) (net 3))
 (segment (start 17.1615 23.586) (end 16.693634 23.586) (width 0.25) (layer F.Cu) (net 3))
 (segment (start 16.602634 23.495) (end 16.383 23.495) (width 0.25) (layer F.Cu) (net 3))
 (segment (start 16.9925 12.1665) (end 17.018 12.192) (width 0.25) (layer F.Cu) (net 41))
 (segment (start 15.494 12.1665) (end 16.9925 12.1665) (width 0.25) (layer F.Cu) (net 41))
 (segment (start 15.474 18.69041) (end 16.38441 17.78) (width 0.25) (layer F.Cu) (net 41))
 (segment (start 15.474 19.3985) (end 15.474 18.69041) (width 0.25) (layer F.Cu) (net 41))
 (segment (start 17.81801 17.229824) (end 17.81801 12.23001) (width 0.25) (layer F.Cu) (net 41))
 (segment (start 17.267834 17.78) (end 17.81801 17.229824) (width 0.25) (layer F.Cu) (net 41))
 (segment (start 16.38441 17.78) (end 17.267834 17.78) (width 0.25) (layer F.Cu) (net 41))
 (segment (start 19.291 12.192) (end 19.304 12.179) (width 0.25) (layer F.Cu) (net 41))
 (segment (start 17.018 12.192) (end 19.291 12.192) (width 0.25) (layer F.Cu) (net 41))
 (segment (start 10.447 20.086) (end 10.427 20.066) (width 0.25) (layer F.Cu) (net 35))
 (segment (start 12.2865 20.086) (end 10.447 20.086) (width 0.25) (layer F.Cu) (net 35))
 (segment (start 16.474 19.3985) (end 16.474 19.049388) (width 0.25) (layer F.Cu) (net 35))
 (segment (start 17.493667 18.826987) (end 19.304 17.016654) (width 0.25) (layer F.Cu) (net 35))
 (segment (start 16.6964 18.826988) (end 17.493667 18.826987) (width 0.25) (layer F.Cu) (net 35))
 (segment (start 19.304 17.016654) (end 19.304 16.777) (width 0.25) (layer F.Cu) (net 35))
 (segment (start 16.474 19.049388) (end 16.6964 18.826988) (width 0.25) (layer F.Cu) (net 35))
 (segment (start 12.699 20.086) (end 12.2865 20.086) (width 0.25) (layer F.Cu) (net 35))
 (segment (start 12.74901 20.13601) (end 12.699 20.086) (width 0.25) (layer F.Cu) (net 35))
 (segment (start 16.204356 20.13601) (end 12.74901 20.13601) (width 0.25) (layer F.Cu) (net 35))
 (segment (start 16.474 19.866366) (end 16.204356 20.13601) (width 0.25) (layer F.Cu) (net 35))
 (segment (start 16.474 19.3985) (end 16.474 19.866366) (width 0.25) (layer F.Cu) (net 35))
 (segment (start 14.474 25.645) (end 13.97 26.149) (width 0.25) (layer F.Cu) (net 35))
 (segment (start 14.474 24.2735) (end 14.474 25.645) (width 0.25) (layer F.Cu) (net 35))
 (segment (start 10.455 23.086) (end 10.427 23.114) (width 0.25) (layer F.Cu) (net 37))
 (segment (start 12.2865 23.086) (end 10.455 23.086) (width 0.25) (layer F.Cu) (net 37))
 (segment (start 13.97 12.2175) (end 12.446 13.7415) (width 0.25) (layer F.Cu) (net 55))
 (segment (start 13.97 12.179) (end 13.97 12.2175) (width 0.25) (layer F.Cu) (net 55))
 (segment (start 12.4335 12.179) (end 12.446 12.1665) (width 0.25) (layer F.Cu) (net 53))
 (segment (start 10.922 12.179) (end 12.4335 12.179) (width 0.25) (layer F.Cu) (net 53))
 (segment (start 12.446 10.922) (end 12.446 12.1665) (width 0.5) (layer F.Cu) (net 53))
 (segment (start 15.494 7.874) (end 12.446 10.922) (width 0.5) (layer F.Cu) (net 53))
 (segment (start 15.494 4.572) (end 15.494 7.874) (width 0.5) (layer F.Cu) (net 53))
 (segment (start 15.4685 57.023) (end 14.986 57.023) (width 0.25) (layer F.Cu) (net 34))
 (segment (start 15.494 56.9975) (end 15.4685 57.023) (width 0.25) (layer F.Cu) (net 34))
 (segment (start 15.494 55.3975) (end 15.494 56.9975) (width 0.25) (layer F.Cu) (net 34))
 (segment (start 17.13 56.9365) (end 17.0435 57.023) (width 0.25) (layer F.Cu) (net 54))
 (segment (start 17.13 55.356) (end 17.13 56.9365) (width 0.25) (layer F.Cu) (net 54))
 (segment (start 10.668 17.227) (end 10.668 16.827) (width 0.25) (layer F.Cu) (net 38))
 (segment (start 11.443019 18.002019) (end 10.668 17.227) (width 0.25) (layer F.Cu) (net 38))
 (segment (start 12.563042 18.00202) (end 11.443019 18.002019) (width 0.25) (layer F.Cu) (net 38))
 (segment (start 13.474 18.912978) (end 12.563042 18.00202) (width 0.25) (layer F.Cu) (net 38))
 (segment (start 13.474 19.3985) (end 13.474 18.912978) (width 0.25) (layer F.Cu) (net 38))
 (segment (start 15.7225 25.4255) (end 15.7225 26.162) (width 0.25) (layer F.Cu) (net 48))
 (segment (start 15.474 25.177) (end 15.7225 25.4255) (width 0.25) (layer F.Cu) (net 48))
 (segment (start 15.474 24.2735) (end 15.474 25.177) (width 0.25) (layer F.Cu) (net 48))
 (segment (start 17.414 26.2785) (end 17.2975 26.162) (width 0.25) (layer F.Cu) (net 52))
 (segment (start 13.944 16.777) (end 13.957 16.764) (width 0.25) (layer F.Cu) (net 39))
 (segment (start 12.446 16.777) (end 13.944 16.777) (width 0.25) (layer F.Cu) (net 39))
 (segment (start 13.9445 16.7515) (end 13.957 16.764) (width 0.25) (layer F.Cu) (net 39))
 (segment (start 13.9445 15.24) (end 13.9445 16.7515) (width 0.25) (layer F.Cu) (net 39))
 (segment (start 13.97 15.2145) (end 13.9445 15.24) (width 0.25) (layer F.Cu) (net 39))
 (segment (start 13.97 13.729) (end 13.97 15.2145) (width 0.25) (layer F.Cu) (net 39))
 (segment (start 14.474 19.3985) (end 14.474 18.546) (width 0.25) (layer F.Cu) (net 39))
 (segment (start 13.957 18.029) (end 13.957 16.764) (width 0.25) (layer F.Cu) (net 39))
 (segment (start 14.474 18.546) (end 13.957 18.029) (width 0.25) (layer F.Cu) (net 39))
 (segment (start 15.5195 16.7515) (end 15.507 16.764) (width 0.25) (layer F.Cu) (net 40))
 (segment (start 15.5195 15.24) (end 15.5195 16.7515) (width 0.25) (layer F.Cu) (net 40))
 (segment (start 17.005 16.764) (end 17.018 16.777) (width 0.25) (layer F.Cu) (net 40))
 (segment (start 15.507 16.764) (end 17.005 16.764) (width 0.25) (layer F.Cu) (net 40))
 (segment (start 15.494 14.318056) (end 15.494 13.7415) (width 0.25) (layer F.Cu) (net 40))
 (segment (start 15.494 15.2145) (end 15.494 14.318056) (width 0.25) (layer F.Cu) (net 40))
 (segment (start 15.5195 15.24) (end 15.494 15.2145) (width 0.25) (layer F.Cu) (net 40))
 (segment (start 14.974 19.3985) (end 14.974 18.554) (width 0.25) (layer F.Cu) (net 40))
 (segment (start 15.507 18.021) (end 15.507 16.764) (width 0.25) (layer F.Cu) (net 40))
 (segment (start 14.974 18.554) (end 15.507 18.021) (width 0.25) (layer F.Cu) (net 40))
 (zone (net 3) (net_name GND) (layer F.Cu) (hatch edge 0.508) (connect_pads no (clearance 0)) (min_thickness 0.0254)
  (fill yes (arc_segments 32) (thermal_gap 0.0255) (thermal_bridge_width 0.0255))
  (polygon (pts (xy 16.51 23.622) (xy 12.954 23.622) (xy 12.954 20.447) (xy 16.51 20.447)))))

